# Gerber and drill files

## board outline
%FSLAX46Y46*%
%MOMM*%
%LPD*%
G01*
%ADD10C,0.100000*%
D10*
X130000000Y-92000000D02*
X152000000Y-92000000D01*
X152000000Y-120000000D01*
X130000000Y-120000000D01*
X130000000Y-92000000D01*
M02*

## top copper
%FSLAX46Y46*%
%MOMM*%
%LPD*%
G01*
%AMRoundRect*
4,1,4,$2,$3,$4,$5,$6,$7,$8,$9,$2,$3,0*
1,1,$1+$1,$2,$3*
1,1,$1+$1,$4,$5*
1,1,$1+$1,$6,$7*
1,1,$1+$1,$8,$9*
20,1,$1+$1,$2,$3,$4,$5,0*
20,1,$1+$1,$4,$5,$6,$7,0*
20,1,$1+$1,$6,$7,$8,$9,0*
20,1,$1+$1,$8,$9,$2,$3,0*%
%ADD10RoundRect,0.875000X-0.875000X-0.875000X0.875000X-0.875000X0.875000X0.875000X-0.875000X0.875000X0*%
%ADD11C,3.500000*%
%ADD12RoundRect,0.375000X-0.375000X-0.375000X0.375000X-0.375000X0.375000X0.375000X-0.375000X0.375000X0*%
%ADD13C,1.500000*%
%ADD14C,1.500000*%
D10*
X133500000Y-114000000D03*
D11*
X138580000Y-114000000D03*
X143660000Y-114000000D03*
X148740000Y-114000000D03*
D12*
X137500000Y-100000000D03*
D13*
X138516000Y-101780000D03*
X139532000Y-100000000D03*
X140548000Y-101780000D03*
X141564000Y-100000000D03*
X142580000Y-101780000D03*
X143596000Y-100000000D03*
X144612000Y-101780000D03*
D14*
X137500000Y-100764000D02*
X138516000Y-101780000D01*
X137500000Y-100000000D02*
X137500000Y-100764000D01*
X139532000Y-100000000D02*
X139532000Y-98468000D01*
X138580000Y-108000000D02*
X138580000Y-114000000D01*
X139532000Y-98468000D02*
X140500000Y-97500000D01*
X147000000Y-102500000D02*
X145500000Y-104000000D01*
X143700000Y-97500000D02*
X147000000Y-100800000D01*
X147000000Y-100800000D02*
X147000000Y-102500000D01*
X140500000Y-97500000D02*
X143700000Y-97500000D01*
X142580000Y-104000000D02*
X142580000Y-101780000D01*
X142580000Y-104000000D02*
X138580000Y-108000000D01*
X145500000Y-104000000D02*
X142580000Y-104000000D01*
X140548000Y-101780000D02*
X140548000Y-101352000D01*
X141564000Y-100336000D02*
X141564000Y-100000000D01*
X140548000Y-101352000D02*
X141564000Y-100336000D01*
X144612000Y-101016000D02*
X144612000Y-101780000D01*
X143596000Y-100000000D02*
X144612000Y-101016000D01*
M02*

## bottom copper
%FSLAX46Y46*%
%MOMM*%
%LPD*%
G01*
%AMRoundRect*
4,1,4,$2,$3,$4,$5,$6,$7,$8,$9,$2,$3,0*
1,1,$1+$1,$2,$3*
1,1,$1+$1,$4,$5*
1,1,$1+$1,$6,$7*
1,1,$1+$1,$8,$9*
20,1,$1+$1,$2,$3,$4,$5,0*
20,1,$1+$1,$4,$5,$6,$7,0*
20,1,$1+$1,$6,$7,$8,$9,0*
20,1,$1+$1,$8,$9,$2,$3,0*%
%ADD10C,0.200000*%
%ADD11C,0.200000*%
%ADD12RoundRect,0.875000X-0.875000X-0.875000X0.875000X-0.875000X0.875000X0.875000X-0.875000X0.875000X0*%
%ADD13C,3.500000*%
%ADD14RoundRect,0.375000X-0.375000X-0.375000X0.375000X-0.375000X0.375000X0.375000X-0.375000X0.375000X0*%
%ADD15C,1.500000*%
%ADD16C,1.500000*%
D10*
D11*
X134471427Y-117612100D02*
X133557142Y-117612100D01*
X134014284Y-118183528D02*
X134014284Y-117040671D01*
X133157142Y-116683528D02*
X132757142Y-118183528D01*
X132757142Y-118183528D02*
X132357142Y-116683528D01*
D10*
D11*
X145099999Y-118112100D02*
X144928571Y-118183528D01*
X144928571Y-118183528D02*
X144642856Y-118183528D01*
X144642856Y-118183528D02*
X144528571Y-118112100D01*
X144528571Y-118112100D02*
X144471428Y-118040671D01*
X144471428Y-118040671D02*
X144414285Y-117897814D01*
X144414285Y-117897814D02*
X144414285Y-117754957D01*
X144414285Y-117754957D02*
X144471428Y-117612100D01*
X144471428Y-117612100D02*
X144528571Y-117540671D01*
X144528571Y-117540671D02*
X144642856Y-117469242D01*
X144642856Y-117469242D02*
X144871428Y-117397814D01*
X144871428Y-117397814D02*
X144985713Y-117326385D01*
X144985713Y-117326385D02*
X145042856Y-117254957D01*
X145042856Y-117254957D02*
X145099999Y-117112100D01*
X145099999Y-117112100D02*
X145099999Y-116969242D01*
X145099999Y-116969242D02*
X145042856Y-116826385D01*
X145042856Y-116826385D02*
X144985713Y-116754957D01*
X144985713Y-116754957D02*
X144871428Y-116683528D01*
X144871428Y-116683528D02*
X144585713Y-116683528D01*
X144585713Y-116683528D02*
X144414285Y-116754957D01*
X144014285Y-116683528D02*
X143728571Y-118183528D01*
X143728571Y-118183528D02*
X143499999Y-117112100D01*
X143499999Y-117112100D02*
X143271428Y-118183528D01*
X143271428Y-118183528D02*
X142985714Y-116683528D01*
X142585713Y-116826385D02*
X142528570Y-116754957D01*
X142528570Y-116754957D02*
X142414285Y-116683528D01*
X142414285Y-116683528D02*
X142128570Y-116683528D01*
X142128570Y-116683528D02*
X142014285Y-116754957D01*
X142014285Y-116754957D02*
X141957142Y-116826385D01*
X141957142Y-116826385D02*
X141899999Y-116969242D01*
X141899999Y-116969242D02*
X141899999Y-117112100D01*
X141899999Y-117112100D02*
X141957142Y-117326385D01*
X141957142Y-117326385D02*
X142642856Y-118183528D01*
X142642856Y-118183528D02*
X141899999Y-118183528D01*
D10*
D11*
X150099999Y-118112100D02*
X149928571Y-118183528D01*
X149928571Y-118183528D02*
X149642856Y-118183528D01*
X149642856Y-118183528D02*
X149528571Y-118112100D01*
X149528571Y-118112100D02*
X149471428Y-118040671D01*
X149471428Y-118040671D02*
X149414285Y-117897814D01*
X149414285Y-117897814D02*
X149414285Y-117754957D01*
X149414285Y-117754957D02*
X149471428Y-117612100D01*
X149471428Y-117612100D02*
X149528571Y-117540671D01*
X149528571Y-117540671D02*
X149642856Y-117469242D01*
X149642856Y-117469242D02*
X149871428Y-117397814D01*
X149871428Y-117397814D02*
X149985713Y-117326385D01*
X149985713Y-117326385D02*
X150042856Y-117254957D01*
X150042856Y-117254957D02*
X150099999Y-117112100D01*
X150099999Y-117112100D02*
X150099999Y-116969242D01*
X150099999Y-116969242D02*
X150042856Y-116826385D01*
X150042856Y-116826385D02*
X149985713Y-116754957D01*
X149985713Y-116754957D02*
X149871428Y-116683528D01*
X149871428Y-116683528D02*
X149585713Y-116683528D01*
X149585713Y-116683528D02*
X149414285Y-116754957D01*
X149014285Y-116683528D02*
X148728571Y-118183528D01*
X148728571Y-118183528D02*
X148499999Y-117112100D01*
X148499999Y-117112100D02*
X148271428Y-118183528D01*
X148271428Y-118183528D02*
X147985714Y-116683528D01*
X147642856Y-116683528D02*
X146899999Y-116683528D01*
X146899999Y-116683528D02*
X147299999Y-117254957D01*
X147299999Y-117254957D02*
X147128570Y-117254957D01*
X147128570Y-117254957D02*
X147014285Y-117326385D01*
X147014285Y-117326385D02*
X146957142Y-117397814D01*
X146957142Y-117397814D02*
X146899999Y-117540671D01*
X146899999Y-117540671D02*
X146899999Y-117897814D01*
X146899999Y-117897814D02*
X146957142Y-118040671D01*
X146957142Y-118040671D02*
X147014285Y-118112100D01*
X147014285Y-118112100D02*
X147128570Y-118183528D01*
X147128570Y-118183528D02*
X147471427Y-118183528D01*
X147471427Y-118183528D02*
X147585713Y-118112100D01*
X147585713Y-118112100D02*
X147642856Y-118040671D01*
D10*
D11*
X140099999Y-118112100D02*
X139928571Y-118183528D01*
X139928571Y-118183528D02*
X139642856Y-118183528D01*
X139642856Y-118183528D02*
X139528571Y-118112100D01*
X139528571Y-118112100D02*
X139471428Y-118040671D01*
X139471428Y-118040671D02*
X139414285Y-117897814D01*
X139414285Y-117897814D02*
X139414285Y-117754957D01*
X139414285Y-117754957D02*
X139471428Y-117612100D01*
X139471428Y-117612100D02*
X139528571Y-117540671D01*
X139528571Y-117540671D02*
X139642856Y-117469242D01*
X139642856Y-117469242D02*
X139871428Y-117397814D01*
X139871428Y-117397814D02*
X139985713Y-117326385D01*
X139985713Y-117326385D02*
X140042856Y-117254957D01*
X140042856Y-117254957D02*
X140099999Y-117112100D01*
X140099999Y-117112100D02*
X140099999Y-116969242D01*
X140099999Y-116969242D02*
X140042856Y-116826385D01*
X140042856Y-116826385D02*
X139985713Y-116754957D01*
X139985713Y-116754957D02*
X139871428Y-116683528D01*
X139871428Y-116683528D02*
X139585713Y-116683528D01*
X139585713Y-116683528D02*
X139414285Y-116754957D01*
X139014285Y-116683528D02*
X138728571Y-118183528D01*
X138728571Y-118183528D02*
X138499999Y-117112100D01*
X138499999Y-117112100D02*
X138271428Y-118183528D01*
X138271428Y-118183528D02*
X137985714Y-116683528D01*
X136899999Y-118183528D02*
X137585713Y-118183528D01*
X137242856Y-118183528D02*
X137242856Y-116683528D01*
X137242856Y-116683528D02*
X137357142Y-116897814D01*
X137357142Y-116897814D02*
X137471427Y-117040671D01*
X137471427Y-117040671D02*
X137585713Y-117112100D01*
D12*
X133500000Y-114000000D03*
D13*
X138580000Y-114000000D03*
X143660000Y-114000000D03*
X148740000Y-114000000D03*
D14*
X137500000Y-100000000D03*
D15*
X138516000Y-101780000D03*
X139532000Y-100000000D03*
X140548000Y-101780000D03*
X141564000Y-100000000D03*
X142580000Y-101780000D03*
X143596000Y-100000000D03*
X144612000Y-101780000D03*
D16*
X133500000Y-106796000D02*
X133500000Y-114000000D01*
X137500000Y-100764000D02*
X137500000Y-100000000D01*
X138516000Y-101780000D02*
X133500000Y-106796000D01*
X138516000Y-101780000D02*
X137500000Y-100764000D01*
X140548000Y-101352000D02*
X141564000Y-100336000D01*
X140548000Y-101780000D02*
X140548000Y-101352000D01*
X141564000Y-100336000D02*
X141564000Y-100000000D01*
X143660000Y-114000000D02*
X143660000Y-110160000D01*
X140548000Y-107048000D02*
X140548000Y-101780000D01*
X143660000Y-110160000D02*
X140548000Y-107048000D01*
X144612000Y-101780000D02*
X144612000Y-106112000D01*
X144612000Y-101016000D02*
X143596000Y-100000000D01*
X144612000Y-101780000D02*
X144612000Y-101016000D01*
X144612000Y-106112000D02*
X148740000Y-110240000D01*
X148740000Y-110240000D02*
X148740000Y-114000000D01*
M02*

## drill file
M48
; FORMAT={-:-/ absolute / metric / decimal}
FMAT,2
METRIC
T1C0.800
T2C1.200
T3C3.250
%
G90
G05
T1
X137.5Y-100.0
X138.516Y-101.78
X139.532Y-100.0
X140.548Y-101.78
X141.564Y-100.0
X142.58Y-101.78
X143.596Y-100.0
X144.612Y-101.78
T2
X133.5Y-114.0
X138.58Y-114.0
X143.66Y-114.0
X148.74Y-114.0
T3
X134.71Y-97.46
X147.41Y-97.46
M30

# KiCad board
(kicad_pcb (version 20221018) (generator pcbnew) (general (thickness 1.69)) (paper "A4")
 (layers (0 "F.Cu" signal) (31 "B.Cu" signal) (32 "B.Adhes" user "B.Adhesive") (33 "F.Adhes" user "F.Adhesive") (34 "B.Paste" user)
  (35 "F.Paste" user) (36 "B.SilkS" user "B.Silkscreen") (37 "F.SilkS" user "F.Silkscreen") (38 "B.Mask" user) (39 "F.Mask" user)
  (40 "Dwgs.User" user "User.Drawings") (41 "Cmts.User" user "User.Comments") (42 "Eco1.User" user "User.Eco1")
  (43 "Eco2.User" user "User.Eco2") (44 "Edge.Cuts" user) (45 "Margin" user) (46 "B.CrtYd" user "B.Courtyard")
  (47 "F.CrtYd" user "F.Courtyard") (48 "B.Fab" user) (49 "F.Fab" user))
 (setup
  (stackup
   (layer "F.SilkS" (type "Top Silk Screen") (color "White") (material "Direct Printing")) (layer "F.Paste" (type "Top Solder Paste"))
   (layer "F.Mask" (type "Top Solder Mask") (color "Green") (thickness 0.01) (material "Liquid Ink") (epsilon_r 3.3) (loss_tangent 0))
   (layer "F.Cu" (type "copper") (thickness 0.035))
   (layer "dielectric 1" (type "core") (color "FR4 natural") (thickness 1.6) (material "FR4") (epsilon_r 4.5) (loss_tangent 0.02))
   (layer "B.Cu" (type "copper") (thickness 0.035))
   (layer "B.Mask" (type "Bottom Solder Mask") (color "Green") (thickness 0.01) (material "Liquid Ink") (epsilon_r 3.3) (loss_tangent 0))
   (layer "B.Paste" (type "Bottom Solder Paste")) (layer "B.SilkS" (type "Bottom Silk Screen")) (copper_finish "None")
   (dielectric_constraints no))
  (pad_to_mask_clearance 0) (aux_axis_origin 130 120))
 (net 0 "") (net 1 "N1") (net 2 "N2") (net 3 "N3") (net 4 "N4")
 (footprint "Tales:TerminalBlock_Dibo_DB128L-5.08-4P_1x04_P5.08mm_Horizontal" (layer "F.Cu") (at 133.5 114)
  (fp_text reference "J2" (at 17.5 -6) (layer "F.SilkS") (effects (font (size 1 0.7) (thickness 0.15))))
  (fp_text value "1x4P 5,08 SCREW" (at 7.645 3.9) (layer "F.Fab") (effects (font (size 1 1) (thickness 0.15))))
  (pad "1" thru_hole roundrect (at 0 0) (size 3.5 3.5) (drill 1.2) (layers "*.Cu" "*.Mask") (roundrect_rratio 0.25) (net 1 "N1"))
  (pad "2" thru_hole circle (at 5.08 0) (size 3.5 3.5) (drill 1.2) (layers "*.Cu" "*.Mask") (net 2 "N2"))
  (pad "3" thru_hole circle (at 10.16 0) (size 3.5 3.5) (drill 1.2) (layers "*.Cu" "*.Mask") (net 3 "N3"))
  (pad "4" thru_hole circle (at 15.24 0) (size 3.5 3.5) (drill 1.2) (layers "*.Cu" "*.Mask") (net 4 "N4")))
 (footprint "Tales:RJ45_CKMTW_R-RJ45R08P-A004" (layer "F.Cu") (at 137.5 100 180)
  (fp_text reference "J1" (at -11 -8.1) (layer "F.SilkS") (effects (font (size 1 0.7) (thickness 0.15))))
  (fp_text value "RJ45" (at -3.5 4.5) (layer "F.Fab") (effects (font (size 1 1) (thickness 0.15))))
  (pad "" np_thru_hole circle (at -9.91 2.54) (size 3.25 3.25) (drill 3.25) (layers "*.Cu" "*.Mask"))
  (pad "" np_thru_hole circle (at 2.79 2.54) (size 3.25 3.25) (drill 3.25) (layers "*.Cu" "*.Mask"))
  (pad "1" thru_hole roundrect (at 0 0) (size 1.5 1.5) (drill 0.8) (layers "*.Cu" "*.Mask") (roundrect_rratio 0.25) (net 1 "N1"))
  (pad "2" thru_hole circle (at -1.016 -1.78) (size 1.5 1.5) (drill 0.8) (layers "*.Cu" "*.Mask") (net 1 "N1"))
  (pad "3" thru_hole circle (at -2.032 0) (size 1.5 1.5) (drill 0.8) (layers "*.Cu" "*.Mask") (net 2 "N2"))
  (pad "4" thru_hole circle (at -3.048 -1.78) (size 1.5 1.5) (drill 0.8) (layers "*.Cu" "*.Mask") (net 3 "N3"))
  (pad "5" thru_hole circle (at -4.064 0) (size 1.5 1.5) (drill 0.8) (layers "*.Cu" "*.Mask") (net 3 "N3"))
  (pad "6" thru_hole circle (at -5.08 -1.78) (size 1.5 1.5) (drill 0.8) (layers "*.Cu" "*.Mask") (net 2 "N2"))
  (pad "7" thru_hole circle (at -6.096 0) (size 1.5 1.5) (drill 0.8) (layers "*.Cu" "*.Mask") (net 4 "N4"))
  (pad "8" thru_hole circle (at -7.112 -1.78) (size 1.5 1.5) (drill 0.8) (layers "*.Cu" "*.Mask") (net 4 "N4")))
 (gr_rect (start 130 92) (end 152 120) (stroke (width 0.1) (type default)) (fill none) (layer "Edge.Cuts"))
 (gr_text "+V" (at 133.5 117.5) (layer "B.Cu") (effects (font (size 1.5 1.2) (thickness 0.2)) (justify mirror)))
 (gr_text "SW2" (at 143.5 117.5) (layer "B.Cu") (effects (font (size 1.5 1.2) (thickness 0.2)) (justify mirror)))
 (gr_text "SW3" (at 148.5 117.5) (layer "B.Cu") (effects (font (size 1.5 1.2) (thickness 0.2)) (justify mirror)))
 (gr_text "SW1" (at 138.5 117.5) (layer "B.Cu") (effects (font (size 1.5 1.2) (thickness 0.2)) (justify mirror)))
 (segment (start 137.5 100.764) (end 138.516 101.78) (width 1.5) (layer "F.Cu") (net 1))
 (segment (start 137.5 100) (end 137.5 100.764) (width 1.5) (layer "F.Cu") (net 1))
 (segment (start 133.5 106.796) (end 133.5 114) (width 1.5) (layer "B.Cu") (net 1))
 (segment (start 137.5 100.764) (end 137.5 100) (width 1.5) (layer "B.Cu") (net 1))
 (segment (start 138.516 101.78) (end 133.5 106.796) (width 1.5) (layer "B.Cu") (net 1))
 (segment (start 138.516 101.78) (end 137.5 100.764) (width 1.5) (layer "B.Cu") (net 1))
 (segment (start 139.532 100) (end 139.532 98.468) (width 1.5) (layer "F.Cu") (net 2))
 (segment (start 138.58 108) (end 138.58 114) (width 1.5) (layer "F.Cu") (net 2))
 (segment (start 139.532 98.468) (end 140.5 97.5) (width 1.5) (layer "F.Cu") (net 2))
 (segment (start 147 102.5) (end 145.5 104) (width 1.5) (layer "F.Cu") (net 2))
 (segment (start 143.7 97.5) (end 147 100.8) (width 1.5) (layer "F.Cu") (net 2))
 (segment (start 147 100.8) (end 147 102.5) (width 1.5) (layer "F.Cu") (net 2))
 (segment (start 140.5 97.5) (end 143.7 97.5) (width 1.5) (layer "F.Cu") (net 2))
 (segment (start 142.58 104) (end 142.58 101.78) (width 1.5) (layer "F.Cu") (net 2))
 (segment (start 142.58 104) (end 138.58 108) (width 1.5) (layer "F.Cu") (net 2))
 (segment (start 145.5 104) (end 142.58 104) (width 1.5) (layer "F.Cu") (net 2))
 (segment (start 140.548 101.78) (end 140.548 101.352) (width 1.5) (layer "F.Cu") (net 3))
 (segment (start 141.564 100.336) (end 141.564 100) (width 1.5) (layer "F.Cu") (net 3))
 (segment (start 140.548 101.352) (end 141.564 100.336) (width 1.5) (layer "F.Cu") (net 3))
 (segment (start 140.548 101.352) (end 141.564 100.336) (width 1.5) (layer "B.Cu") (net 3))
 (segment (start 140.548 101.78) (end 140.548 101.352) (width 1.5) (layer "B.Cu") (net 3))
 (segment (start 141.564 100.336) (end 141.564 100) (width 1.5) (layer "B.Cu") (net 3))
 (segment (start 143.66 114) (end 143.66 110.16) (width 1.5) (layer "B.Cu") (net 3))
 (segment (start 140.548 107.048) (end 140.548 101.78) (width 1.5) (layer "B.Cu") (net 3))
 (segment (start 143.66 110.16) (end 140.548 107.048) (width 1.5) (layer "B.Cu") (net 3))
 (segment (start 144.612 101.016) (end 144.612 101.78) (width 1.5) (layer "F.Cu") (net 4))
 (segment (start 143.596 100) (end 144.612 101.016) (width 1.5) (layer "F.Cu") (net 4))
 (segment (start 144.612 101.78) (end 144.612 106.112) (width 1.5) (layer "B.Cu") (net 4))
 (segment (start 144.612 101.016) (end 143.596 100) (width 1.5) (layer "B.Cu") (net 4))
 (segment (start 144.612 101.78) (end 144.612 101.016) (width 1.5) (layer "B.Cu") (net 4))
 (segment (start 144.612 106.112) (end 148.74 110.24) (width 1.5) (layer "B.Cu") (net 4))
 (segment (start 148.74 110.24) (end 148.74 114) (width 1.5) (layer "B.Cu") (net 4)))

